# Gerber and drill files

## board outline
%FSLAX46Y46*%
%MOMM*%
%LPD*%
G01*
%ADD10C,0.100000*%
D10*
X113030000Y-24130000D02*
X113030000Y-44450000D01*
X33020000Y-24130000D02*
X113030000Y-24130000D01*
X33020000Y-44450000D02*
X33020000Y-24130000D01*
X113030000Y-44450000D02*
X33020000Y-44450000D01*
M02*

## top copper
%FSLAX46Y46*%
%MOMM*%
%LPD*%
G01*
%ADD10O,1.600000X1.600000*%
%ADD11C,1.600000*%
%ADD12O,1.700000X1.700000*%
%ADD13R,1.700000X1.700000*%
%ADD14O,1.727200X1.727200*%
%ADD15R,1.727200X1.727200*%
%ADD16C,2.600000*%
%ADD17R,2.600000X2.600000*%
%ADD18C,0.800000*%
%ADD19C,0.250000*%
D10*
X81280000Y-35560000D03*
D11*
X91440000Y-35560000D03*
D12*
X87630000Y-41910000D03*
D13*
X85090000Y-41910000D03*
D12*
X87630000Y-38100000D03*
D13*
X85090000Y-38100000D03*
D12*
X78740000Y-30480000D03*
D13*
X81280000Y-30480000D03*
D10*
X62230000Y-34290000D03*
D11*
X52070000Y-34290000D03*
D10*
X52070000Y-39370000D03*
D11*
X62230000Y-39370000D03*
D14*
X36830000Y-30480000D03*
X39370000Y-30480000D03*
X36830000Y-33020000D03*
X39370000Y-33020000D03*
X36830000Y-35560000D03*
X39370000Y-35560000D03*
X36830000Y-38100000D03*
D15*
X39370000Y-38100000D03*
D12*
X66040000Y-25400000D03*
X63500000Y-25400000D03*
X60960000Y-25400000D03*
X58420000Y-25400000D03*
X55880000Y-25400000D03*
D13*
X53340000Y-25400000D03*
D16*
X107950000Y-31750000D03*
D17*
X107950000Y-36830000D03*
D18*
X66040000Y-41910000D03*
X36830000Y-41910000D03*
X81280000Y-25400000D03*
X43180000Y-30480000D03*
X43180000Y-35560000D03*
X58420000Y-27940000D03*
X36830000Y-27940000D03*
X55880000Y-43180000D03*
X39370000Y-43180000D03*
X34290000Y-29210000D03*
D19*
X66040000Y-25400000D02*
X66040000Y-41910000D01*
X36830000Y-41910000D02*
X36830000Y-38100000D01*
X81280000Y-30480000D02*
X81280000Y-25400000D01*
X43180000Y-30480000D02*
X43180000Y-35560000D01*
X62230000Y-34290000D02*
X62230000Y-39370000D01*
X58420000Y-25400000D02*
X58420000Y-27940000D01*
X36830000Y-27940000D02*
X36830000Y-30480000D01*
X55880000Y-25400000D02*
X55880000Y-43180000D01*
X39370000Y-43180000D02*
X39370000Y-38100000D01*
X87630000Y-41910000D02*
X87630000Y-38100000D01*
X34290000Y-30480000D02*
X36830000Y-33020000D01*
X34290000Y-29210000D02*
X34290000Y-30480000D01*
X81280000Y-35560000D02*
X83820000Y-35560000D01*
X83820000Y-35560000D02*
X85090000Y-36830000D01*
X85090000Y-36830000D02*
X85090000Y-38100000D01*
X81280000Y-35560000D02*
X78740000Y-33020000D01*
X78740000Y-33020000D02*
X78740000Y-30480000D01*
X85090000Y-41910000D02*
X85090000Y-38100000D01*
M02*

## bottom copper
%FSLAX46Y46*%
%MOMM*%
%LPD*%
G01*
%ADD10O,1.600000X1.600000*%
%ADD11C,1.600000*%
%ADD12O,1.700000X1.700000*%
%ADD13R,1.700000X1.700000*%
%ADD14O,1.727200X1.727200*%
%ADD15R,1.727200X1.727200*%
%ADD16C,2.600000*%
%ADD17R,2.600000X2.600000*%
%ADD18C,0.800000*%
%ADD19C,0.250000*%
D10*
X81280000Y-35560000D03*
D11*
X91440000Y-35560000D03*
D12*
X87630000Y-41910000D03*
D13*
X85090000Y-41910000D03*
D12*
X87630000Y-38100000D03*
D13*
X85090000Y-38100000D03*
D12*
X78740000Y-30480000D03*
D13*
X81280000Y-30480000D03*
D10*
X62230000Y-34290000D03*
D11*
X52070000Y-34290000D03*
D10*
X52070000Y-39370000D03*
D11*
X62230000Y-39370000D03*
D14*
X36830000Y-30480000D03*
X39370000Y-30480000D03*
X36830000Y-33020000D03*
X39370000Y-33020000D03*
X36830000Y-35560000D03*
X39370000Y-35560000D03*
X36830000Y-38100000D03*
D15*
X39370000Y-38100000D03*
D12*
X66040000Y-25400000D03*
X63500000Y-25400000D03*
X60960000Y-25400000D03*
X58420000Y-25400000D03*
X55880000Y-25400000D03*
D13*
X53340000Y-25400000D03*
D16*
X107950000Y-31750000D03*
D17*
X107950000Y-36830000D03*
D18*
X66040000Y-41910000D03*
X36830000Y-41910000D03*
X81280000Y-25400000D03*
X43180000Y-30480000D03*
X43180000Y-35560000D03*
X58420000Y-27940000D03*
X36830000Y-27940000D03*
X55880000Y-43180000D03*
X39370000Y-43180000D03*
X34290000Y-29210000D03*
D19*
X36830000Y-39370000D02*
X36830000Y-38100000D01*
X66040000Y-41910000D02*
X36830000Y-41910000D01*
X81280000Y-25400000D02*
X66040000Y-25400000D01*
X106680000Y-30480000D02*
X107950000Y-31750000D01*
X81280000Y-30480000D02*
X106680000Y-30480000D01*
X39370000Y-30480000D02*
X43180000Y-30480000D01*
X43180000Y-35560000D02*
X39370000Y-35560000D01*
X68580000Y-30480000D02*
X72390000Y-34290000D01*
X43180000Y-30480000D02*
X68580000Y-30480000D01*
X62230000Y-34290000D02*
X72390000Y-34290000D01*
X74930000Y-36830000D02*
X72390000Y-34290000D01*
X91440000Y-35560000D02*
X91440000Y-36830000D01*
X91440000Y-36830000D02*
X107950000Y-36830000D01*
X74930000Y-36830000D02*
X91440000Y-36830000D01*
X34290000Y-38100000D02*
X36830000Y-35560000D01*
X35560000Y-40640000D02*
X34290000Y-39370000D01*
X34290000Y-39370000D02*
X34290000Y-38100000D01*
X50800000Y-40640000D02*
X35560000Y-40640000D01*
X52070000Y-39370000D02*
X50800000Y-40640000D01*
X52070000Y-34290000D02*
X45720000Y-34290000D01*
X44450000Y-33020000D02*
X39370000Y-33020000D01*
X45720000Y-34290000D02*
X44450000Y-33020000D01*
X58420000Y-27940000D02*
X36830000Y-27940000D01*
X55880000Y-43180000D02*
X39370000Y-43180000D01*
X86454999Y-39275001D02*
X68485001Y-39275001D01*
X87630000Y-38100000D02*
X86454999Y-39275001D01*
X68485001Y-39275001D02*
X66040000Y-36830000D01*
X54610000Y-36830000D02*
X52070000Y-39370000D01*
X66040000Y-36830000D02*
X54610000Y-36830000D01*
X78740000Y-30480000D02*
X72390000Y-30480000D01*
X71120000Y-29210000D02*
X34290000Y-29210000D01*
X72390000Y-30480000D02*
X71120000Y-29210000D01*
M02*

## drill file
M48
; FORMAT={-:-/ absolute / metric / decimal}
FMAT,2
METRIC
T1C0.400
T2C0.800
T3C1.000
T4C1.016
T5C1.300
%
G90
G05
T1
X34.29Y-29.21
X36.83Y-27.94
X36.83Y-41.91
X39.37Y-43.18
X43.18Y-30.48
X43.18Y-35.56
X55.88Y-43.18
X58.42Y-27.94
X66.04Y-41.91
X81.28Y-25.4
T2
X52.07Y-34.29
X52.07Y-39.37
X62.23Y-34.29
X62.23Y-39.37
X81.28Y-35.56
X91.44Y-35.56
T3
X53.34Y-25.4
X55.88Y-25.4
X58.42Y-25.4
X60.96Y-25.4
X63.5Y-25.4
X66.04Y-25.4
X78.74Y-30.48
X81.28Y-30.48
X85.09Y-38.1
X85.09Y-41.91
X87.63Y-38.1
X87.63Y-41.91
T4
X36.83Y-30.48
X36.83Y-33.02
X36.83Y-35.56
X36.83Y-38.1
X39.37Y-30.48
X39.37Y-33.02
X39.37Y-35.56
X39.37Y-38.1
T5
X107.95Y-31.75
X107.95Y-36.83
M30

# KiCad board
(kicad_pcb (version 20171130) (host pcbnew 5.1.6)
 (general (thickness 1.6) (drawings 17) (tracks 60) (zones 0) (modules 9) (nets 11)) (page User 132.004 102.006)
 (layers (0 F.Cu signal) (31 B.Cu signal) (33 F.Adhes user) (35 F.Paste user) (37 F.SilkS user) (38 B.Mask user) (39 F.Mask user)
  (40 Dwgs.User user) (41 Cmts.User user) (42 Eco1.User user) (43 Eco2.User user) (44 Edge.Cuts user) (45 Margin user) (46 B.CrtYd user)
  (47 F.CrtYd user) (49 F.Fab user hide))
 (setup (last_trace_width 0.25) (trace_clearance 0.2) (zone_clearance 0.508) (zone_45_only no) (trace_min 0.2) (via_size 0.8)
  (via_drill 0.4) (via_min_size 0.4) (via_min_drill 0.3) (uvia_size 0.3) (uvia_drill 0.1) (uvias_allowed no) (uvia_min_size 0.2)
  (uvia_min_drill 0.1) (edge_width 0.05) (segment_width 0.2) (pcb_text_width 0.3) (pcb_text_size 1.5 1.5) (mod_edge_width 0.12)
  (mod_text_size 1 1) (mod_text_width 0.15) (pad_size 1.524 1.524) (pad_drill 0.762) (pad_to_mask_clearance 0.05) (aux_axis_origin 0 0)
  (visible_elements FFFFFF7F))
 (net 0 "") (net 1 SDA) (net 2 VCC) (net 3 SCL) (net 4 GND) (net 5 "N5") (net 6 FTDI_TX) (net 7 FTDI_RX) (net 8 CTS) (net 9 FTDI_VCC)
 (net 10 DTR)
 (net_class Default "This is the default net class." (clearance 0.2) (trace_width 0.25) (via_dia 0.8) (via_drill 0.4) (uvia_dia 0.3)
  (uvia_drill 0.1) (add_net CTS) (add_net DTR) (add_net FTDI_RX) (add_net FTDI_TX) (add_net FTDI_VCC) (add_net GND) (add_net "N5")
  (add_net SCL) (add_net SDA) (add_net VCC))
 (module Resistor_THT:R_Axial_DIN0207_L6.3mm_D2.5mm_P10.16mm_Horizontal (layer F.Cu) (at 91.44 35.56 180)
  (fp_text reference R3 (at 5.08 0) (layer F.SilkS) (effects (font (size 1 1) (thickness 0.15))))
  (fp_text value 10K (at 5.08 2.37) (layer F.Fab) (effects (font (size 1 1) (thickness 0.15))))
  (pad 2 thru_hole oval (at 10.16 0 180) (size 1.6 1.6) (drill 0.8) (layers *.Cu *.Mask) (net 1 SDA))
  (pad 1 thru_hole circle (at 0 0 180) (size 1.6 1.6) (drill 0.8) (layers *.Cu *.Mask) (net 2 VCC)))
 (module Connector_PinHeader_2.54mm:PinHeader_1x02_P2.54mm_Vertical (layer F.Cu) (at 85.09 41.91 90)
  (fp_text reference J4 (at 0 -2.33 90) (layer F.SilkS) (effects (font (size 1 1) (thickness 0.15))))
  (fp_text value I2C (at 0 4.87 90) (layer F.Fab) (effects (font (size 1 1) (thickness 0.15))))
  (pad 2 thru_hole oval (at 0 2.54 90) (size 1.7 1.7) (drill 1) (layers *.Cu *.Mask) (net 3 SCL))
  (pad 1 thru_hole rect (at 0 0 90) (size 1.7 1.7) (drill 1) (layers *.Cu *.Mask) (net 1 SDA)))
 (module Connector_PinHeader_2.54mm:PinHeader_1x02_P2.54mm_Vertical (layer F.Cu) (at 85.09 38.1 90)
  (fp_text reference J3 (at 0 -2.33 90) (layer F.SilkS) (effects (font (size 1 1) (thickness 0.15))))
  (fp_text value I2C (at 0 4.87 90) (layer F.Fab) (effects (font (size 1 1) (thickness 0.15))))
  (pad 2 thru_hole oval (at 0 2.54 90) (size 1.7 1.7) (drill 1) (layers *.Cu *.Mask) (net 3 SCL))
  (pad 1 thru_hole rect (at 0 0 90) (size 1.7 1.7) (drill 1) (layers *.Cu *.Mask) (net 1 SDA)))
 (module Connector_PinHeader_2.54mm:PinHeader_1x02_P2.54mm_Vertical (layer F.Cu) (at 81.28 30.48 270)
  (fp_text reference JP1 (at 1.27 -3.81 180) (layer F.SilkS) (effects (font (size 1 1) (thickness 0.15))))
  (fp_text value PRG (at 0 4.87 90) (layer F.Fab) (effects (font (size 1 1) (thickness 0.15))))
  (pad 2 thru_hole oval (at 0 2.54 270) (size 1.7 1.7) (drill 1) (layers *.Cu *.Mask) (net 1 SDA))
  (pad 1 thru_hole rect (at 0 0 270) (size 1.7 1.7) (drill 1) (layers *.Cu *.Mask) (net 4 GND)))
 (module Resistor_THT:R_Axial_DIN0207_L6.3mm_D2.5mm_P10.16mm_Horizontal (layer F.Cu) (at 52.07 34.29)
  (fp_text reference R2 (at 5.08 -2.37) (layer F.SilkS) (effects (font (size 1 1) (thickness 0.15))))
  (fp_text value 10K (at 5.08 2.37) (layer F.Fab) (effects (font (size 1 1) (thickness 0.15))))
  (pad 2 thru_hole oval (at 10.16 0) (size 1.6 1.6) (drill 0.8) (layers *.Cu *.Mask) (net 2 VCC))
  (pad 1 thru_hole circle (at 0 0) (size 1.6 1.6) (drill 0.8) (layers *.Cu *.Mask) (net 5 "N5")))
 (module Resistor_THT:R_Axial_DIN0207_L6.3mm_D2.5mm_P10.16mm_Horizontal (layer F.Cu) (at 62.23 39.37 180)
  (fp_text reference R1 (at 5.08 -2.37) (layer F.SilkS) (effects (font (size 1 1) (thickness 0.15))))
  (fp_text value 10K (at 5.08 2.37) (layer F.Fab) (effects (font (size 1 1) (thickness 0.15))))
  (pad 2 thru_hole oval (at 10.16 0 180) (size 1.6 1.6) (drill 0.8) (layers *.Cu *.Mask) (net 3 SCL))
  (pad 1 thru_hole circle (at 0 0 180) (size 1.6 1.6) (drill 0.8) (layers *.Cu *.Mask) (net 2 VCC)))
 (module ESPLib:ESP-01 (layer F.Cu) (at 39.37 38.1 180)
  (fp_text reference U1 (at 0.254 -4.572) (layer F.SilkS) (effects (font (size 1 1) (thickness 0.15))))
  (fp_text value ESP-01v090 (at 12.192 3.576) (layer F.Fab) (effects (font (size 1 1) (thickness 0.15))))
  (pad 8 thru_hole oval (at 2.54 7.62 180) (size 1.7272 1.7272) (drill 1.016) (layers *.Cu *.Mask F.SilkS) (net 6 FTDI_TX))
  (pad 7 thru_hole oval (at 0 7.62 180) (size 1.7272 1.7272) (drill 1.016) (layers *.Cu *.Mask F.SilkS) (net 2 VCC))
  (pad 6 thru_hole oval (at 2.54 5.08 180) (size 1.7272 1.7272) (drill 1.016) (layers *.Cu *.Mask F.SilkS) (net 1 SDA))
  (pad 5 thru_hole oval (at 0 5.08 180) (size 1.7272 1.7272) (drill 1.016) (layers *.Cu *.Mask F.SilkS) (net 5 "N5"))
  (pad 4 thru_hole oval (at 2.54 2.54 180) (size 1.7272 1.7272) (drill 1.016) (layers *.Cu *.Mask F.SilkS) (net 3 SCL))
  (pad 3 thru_hole oval (at 0 2.54 180) (size 1.7272 1.7272) (drill 1.016) (layers *.Cu *.Mask F.SilkS) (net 2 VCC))
  (pad 2 thru_hole oval (at 2.54 0 180) (size 1.7272 1.7272) (drill 1.016) (layers *.Cu *.Mask F.SilkS) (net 4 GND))
  (pad 1 thru_hole rect (at 0 0 180) (size 1.7272 1.7272) (drill 1.016) (layers *.Cu *.Mask F.SilkS) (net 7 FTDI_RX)))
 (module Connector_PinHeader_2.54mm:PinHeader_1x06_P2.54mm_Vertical (layer F.Cu) (at 53.34 25.4 90)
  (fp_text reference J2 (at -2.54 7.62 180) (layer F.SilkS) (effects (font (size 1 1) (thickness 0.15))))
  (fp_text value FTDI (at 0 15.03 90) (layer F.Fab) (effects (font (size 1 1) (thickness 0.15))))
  (pad 6 thru_hole oval (at 0 12.7 90) (size 1.7 1.7) (drill 1) (layers *.Cu *.Mask) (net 4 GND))
  (pad 5 thru_hole oval (at 0 10.16 90) (size 1.7 1.7) (drill 1) (layers *.Cu *.Mask) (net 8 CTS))
  (pad 4 thru_hole oval (at 0 7.62 90) (size 1.7 1.7) (drill 1) (layers *.Cu *.Mask) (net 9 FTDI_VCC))
  (pad 3 thru_hole oval (at 0 5.08 90) (size 1.7 1.7) (drill 1) (layers *.Cu *.Mask) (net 6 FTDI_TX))
  (pad 2 thru_hole oval (at 0 2.54 90) (size 1.7 1.7) (drill 1) (layers *.Cu *.Mask) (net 7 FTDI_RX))
  (pad 1 thru_hole rect (at 0 0 90) (size 1.7 1.7) (drill 1) (layers *.Cu *.Mask) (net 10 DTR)))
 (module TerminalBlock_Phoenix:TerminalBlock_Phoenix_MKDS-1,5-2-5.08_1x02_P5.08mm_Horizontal (layer F.Cu) (at 107.95 36.83 90)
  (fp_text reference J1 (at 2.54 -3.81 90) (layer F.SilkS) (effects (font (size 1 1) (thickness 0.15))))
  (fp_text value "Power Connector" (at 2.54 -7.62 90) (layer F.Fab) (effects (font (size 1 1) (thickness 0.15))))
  (pad 2 thru_hole circle (at 5.08 0 90) (size 2.6 2.6) (drill 1.3) (layers *.Cu *.Mask) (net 4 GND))
  (pad 1 thru_hole rect (at 0 0 90) (size 2.6 2.6) (drill 1.3) (layers *.Cu *.Mask) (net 2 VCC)))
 (gr_line (start 113.03 24.13) (end 113.03 44.45) (layer Edge.Cuts) (width 0.1))
 (gr_line (start 33.02 24.13) (end 113.03 24.13) (layer Edge.Cuts) (width 0.1))
 (gr_line (start 33.02 44.45) (end 33.02 24.13) (layer Edge.Cuts) (width 0.1))
 (gr_line (start 113.03 44.45) (end 33.02 44.45) (layer Edge.Cuts) (width 0.1))
 (segment (start 36.83 39.37) (end 36.83 38.1) (width 0.25) (layer B.Cu) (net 4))
 (segment (start 66.04 25.4) (end 66.04 41.91) (width 0.25) (layer F.Cu) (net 4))
 (via (at 66.04 41.91) (size 0.8) (drill 0.4) (layers F.Cu B.Cu) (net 4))
 (via (at 36.83 41.91) (size 0.8) (drill 0.4) (layers F.Cu B.Cu) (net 4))
 (segment (start 66.04 41.91) (end 36.83 41.91) (width 0.25) (layer B.Cu) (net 4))
 (segment (start 36.83 41.91) (end 36.83 38.1) (width 0.25) (layer F.Cu) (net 4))
 (via (at 81.28 25.4) (size 0.8) (drill 0.4) (layers F.Cu B.Cu) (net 4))
 (segment (start 81.28 30.48) (end 81.28 25.4) (width 0.25) (layer F.Cu) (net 4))
 (segment (start 81.28 25.4) (end 66.04 25.4) (width 0.25) (layer B.Cu) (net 4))
 (segment (start 106.68 30.48) (end 107.95 31.75) (width 0.25) (layer B.Cu) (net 4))
 (segment (start 81.28 30.48) (end 106.68 30.48) (width 0.25) (layer B.Cu) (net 4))
 (via (at 43.18 30.48) (size 0.8) (drill 0.4) (layers F.Cu B.Cu) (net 2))
 (segment (start 39.37 30.48) (end 43.18 30.48) (width 0.25) (layer B.Cu) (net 2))
 (via (at 43.18 35.56) (size 0.8) (drill 0.4) (layers F.Cu B.Cu) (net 2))
 (segment (start 43.18 30.48) (end 43.18 35.56) (width 0.25) (layer F.Cu) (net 2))
 (segment (start 43.18 35.56) (end 39.37 35.56) (width 0.25) (layer B.Cu) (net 2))
 (segment (start 62.23 34.29) (end 62.23 39.37) (width 0.25) (layer F.Cu) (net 2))
 (segment (start 68.58 30.48) (end 72.39 34.29) (width 0.25) (layer B.Cu) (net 2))
 (segment (start 43.18 30.48) (end 68.58 30.48) (width 0.25) (layer B.Cu) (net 2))
 (segment (start 62.23 34.29) (end 72.39 34.29) (width 0.25) (layer B.Cu) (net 2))
 (segment (start 74.93 36.83) (end 72.39 34.29) (width 0.25) (layer B.Cu) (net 2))
 (segment (start 91.44 35.56) (end 91.44 36.83) (width 0.25) (layer B.Cu) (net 2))
 (segment (start 91.44 36.83) (end 107.95 36.83) (width 0.25) (layer B.Cu) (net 2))
 (segment (start 74.93 36.83) (end 91.44 36.83) (width 0.25) (layer B.Cu) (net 2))
 (segment (start 34.29 38.1) (end 36.83 35.56) (width 0.25) (layer B.Cu) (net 3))
 (segment (start 35.56 40.64) (end 34.29 39.37) (width 0.25) (layer B.Cu) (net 3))
 (segment (start 34.29 39.37) (end 34.29 38.1) (width 0.25) (layer B.Cu) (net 3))
 (segment (start 50.8 40.64) (end 35.56 40.64) (width 0.25) (layer B.Cu) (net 3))
 (segment (start 52.07 39.37) (end 50.8 40.64) (width 0.25) (layer B.Cu) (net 3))
 (segment (start 52.07 34.29) (end 45.72 34.29) (width 0.25) (layer B.Cu) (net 5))
 (segment (start 44.45 33.02) (end 39.37 33.02) (width 0.25) (layer B.Cu) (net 5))
 (segment (start 45.72 34.29) (end 44.45 33.02) (width 0.25) (layer B.Cu) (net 5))
 (segment (start 58.42 25.4) (end 58.42 27.94) (width 0.25) (layer F.Cu) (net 6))
 (via (at 58.42 27.94) (size 0.8) (drill 0.4) (layers F.Cu B.Cu) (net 6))
 (via (at 36.83 27.94) (size 0.8) (drill 0.4) (layers F.Cu B.Cu) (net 6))
 (segment (start 58.42 27.94) (end 36.83 27.94) (width 0.25) (layer B.Cu) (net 6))
 (segment (start 36.83 27.94) (end 36.83 30.48) (width 0.25) (layer F.Cu) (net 6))
 (via (at 55.88 43.18) (size 0.8) (drill 0.4) (layers F.Cu B.Cu) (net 7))
 (segment (start 55.88 25.4) (end 55.88 43.18) (width 0.25) (layer F.Cu) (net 7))
 (via (at 39.37 43.18) (size 0.8) (drill 0.4) (layers F.Cu B.Cu) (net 7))
 (segment (start 55.88 43.18) (end 39.37 43.18) (width 0.25) (layer B.Cu) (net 7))
 (segment (start 39.37 43.18) (end 39.37 38.1) (width 0.25) (layer F.Cu) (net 7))
 (segment (start 87.63 41.91) (end 87.63 38.1) (width 0.25) (layer F.Cu) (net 3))
 (segment (start 86.454999 39.275001) (end 68.485001 39.275001) (width 0.25) (layer B.Cu) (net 3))
 (segment (start 87.63 38.1) (end 86.454999 39.275001) (width 0.25) (layer B.Cu) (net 3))
 (segment (start 68.485001 39.275001) (end 66.04 36.83) (width 0.25) (layer B.Cu) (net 3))
 (segment (start 54.61 36.83) (end 52.07 39.37) (width 0.25) (layer B.Cu) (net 3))
 (segment (start 66.04 36.83) (end 54.61 36.83) (width 0.25) (layer B.Cu) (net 3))
 (segment (start 78.74 30.48) (end 72.39 30.48) (width 0.25) (layer B.Cu) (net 1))
 (via (at 34.29 29.21) (size 0.8) (drill 0.4) (layers F.Cu B.Cu) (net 1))
 (segment (start 71.12 29.21) (end 34.29 29.21) (width 0.25) (layer B.Cu) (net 1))
 (segment (start 72.39 30.48) (end 71.12 29.21) (width 0.25) (layer B.Cu) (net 1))
 (segment (start 34.29 30.48) (end 36.83 33.02) (width 0.25) (layer F.Cu) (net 1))
 (segment (start 34.29 29.21) (end 34.29 30.48) (width 0.25) (layer F.Cu) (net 1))
 (segment (start 81.28 35.56) (end 83.82 35.56) (width 0.25) (layer F.Cu) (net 1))
 (segment (start 83.82 35.56) (end 85.09 36.83) (width 0.25) (layer F.Cu) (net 1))
 (segment (start 85.09 36.83) (end 85.09 38.1) (width 0.25) (layer F.Cu) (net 1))
 (segment (start 81.28 35.56) (end 78.74 33.02) (width 0.25) (layer F.Cu) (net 1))
 (segment (start 78.74 33.02) (end 78.74 30.48) (width 0.25) (layer F.Cu) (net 1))
 (segment (start 85.09 41.91) (end 85.09 38.1) (width 0.25) (layer F.Cu) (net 1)))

